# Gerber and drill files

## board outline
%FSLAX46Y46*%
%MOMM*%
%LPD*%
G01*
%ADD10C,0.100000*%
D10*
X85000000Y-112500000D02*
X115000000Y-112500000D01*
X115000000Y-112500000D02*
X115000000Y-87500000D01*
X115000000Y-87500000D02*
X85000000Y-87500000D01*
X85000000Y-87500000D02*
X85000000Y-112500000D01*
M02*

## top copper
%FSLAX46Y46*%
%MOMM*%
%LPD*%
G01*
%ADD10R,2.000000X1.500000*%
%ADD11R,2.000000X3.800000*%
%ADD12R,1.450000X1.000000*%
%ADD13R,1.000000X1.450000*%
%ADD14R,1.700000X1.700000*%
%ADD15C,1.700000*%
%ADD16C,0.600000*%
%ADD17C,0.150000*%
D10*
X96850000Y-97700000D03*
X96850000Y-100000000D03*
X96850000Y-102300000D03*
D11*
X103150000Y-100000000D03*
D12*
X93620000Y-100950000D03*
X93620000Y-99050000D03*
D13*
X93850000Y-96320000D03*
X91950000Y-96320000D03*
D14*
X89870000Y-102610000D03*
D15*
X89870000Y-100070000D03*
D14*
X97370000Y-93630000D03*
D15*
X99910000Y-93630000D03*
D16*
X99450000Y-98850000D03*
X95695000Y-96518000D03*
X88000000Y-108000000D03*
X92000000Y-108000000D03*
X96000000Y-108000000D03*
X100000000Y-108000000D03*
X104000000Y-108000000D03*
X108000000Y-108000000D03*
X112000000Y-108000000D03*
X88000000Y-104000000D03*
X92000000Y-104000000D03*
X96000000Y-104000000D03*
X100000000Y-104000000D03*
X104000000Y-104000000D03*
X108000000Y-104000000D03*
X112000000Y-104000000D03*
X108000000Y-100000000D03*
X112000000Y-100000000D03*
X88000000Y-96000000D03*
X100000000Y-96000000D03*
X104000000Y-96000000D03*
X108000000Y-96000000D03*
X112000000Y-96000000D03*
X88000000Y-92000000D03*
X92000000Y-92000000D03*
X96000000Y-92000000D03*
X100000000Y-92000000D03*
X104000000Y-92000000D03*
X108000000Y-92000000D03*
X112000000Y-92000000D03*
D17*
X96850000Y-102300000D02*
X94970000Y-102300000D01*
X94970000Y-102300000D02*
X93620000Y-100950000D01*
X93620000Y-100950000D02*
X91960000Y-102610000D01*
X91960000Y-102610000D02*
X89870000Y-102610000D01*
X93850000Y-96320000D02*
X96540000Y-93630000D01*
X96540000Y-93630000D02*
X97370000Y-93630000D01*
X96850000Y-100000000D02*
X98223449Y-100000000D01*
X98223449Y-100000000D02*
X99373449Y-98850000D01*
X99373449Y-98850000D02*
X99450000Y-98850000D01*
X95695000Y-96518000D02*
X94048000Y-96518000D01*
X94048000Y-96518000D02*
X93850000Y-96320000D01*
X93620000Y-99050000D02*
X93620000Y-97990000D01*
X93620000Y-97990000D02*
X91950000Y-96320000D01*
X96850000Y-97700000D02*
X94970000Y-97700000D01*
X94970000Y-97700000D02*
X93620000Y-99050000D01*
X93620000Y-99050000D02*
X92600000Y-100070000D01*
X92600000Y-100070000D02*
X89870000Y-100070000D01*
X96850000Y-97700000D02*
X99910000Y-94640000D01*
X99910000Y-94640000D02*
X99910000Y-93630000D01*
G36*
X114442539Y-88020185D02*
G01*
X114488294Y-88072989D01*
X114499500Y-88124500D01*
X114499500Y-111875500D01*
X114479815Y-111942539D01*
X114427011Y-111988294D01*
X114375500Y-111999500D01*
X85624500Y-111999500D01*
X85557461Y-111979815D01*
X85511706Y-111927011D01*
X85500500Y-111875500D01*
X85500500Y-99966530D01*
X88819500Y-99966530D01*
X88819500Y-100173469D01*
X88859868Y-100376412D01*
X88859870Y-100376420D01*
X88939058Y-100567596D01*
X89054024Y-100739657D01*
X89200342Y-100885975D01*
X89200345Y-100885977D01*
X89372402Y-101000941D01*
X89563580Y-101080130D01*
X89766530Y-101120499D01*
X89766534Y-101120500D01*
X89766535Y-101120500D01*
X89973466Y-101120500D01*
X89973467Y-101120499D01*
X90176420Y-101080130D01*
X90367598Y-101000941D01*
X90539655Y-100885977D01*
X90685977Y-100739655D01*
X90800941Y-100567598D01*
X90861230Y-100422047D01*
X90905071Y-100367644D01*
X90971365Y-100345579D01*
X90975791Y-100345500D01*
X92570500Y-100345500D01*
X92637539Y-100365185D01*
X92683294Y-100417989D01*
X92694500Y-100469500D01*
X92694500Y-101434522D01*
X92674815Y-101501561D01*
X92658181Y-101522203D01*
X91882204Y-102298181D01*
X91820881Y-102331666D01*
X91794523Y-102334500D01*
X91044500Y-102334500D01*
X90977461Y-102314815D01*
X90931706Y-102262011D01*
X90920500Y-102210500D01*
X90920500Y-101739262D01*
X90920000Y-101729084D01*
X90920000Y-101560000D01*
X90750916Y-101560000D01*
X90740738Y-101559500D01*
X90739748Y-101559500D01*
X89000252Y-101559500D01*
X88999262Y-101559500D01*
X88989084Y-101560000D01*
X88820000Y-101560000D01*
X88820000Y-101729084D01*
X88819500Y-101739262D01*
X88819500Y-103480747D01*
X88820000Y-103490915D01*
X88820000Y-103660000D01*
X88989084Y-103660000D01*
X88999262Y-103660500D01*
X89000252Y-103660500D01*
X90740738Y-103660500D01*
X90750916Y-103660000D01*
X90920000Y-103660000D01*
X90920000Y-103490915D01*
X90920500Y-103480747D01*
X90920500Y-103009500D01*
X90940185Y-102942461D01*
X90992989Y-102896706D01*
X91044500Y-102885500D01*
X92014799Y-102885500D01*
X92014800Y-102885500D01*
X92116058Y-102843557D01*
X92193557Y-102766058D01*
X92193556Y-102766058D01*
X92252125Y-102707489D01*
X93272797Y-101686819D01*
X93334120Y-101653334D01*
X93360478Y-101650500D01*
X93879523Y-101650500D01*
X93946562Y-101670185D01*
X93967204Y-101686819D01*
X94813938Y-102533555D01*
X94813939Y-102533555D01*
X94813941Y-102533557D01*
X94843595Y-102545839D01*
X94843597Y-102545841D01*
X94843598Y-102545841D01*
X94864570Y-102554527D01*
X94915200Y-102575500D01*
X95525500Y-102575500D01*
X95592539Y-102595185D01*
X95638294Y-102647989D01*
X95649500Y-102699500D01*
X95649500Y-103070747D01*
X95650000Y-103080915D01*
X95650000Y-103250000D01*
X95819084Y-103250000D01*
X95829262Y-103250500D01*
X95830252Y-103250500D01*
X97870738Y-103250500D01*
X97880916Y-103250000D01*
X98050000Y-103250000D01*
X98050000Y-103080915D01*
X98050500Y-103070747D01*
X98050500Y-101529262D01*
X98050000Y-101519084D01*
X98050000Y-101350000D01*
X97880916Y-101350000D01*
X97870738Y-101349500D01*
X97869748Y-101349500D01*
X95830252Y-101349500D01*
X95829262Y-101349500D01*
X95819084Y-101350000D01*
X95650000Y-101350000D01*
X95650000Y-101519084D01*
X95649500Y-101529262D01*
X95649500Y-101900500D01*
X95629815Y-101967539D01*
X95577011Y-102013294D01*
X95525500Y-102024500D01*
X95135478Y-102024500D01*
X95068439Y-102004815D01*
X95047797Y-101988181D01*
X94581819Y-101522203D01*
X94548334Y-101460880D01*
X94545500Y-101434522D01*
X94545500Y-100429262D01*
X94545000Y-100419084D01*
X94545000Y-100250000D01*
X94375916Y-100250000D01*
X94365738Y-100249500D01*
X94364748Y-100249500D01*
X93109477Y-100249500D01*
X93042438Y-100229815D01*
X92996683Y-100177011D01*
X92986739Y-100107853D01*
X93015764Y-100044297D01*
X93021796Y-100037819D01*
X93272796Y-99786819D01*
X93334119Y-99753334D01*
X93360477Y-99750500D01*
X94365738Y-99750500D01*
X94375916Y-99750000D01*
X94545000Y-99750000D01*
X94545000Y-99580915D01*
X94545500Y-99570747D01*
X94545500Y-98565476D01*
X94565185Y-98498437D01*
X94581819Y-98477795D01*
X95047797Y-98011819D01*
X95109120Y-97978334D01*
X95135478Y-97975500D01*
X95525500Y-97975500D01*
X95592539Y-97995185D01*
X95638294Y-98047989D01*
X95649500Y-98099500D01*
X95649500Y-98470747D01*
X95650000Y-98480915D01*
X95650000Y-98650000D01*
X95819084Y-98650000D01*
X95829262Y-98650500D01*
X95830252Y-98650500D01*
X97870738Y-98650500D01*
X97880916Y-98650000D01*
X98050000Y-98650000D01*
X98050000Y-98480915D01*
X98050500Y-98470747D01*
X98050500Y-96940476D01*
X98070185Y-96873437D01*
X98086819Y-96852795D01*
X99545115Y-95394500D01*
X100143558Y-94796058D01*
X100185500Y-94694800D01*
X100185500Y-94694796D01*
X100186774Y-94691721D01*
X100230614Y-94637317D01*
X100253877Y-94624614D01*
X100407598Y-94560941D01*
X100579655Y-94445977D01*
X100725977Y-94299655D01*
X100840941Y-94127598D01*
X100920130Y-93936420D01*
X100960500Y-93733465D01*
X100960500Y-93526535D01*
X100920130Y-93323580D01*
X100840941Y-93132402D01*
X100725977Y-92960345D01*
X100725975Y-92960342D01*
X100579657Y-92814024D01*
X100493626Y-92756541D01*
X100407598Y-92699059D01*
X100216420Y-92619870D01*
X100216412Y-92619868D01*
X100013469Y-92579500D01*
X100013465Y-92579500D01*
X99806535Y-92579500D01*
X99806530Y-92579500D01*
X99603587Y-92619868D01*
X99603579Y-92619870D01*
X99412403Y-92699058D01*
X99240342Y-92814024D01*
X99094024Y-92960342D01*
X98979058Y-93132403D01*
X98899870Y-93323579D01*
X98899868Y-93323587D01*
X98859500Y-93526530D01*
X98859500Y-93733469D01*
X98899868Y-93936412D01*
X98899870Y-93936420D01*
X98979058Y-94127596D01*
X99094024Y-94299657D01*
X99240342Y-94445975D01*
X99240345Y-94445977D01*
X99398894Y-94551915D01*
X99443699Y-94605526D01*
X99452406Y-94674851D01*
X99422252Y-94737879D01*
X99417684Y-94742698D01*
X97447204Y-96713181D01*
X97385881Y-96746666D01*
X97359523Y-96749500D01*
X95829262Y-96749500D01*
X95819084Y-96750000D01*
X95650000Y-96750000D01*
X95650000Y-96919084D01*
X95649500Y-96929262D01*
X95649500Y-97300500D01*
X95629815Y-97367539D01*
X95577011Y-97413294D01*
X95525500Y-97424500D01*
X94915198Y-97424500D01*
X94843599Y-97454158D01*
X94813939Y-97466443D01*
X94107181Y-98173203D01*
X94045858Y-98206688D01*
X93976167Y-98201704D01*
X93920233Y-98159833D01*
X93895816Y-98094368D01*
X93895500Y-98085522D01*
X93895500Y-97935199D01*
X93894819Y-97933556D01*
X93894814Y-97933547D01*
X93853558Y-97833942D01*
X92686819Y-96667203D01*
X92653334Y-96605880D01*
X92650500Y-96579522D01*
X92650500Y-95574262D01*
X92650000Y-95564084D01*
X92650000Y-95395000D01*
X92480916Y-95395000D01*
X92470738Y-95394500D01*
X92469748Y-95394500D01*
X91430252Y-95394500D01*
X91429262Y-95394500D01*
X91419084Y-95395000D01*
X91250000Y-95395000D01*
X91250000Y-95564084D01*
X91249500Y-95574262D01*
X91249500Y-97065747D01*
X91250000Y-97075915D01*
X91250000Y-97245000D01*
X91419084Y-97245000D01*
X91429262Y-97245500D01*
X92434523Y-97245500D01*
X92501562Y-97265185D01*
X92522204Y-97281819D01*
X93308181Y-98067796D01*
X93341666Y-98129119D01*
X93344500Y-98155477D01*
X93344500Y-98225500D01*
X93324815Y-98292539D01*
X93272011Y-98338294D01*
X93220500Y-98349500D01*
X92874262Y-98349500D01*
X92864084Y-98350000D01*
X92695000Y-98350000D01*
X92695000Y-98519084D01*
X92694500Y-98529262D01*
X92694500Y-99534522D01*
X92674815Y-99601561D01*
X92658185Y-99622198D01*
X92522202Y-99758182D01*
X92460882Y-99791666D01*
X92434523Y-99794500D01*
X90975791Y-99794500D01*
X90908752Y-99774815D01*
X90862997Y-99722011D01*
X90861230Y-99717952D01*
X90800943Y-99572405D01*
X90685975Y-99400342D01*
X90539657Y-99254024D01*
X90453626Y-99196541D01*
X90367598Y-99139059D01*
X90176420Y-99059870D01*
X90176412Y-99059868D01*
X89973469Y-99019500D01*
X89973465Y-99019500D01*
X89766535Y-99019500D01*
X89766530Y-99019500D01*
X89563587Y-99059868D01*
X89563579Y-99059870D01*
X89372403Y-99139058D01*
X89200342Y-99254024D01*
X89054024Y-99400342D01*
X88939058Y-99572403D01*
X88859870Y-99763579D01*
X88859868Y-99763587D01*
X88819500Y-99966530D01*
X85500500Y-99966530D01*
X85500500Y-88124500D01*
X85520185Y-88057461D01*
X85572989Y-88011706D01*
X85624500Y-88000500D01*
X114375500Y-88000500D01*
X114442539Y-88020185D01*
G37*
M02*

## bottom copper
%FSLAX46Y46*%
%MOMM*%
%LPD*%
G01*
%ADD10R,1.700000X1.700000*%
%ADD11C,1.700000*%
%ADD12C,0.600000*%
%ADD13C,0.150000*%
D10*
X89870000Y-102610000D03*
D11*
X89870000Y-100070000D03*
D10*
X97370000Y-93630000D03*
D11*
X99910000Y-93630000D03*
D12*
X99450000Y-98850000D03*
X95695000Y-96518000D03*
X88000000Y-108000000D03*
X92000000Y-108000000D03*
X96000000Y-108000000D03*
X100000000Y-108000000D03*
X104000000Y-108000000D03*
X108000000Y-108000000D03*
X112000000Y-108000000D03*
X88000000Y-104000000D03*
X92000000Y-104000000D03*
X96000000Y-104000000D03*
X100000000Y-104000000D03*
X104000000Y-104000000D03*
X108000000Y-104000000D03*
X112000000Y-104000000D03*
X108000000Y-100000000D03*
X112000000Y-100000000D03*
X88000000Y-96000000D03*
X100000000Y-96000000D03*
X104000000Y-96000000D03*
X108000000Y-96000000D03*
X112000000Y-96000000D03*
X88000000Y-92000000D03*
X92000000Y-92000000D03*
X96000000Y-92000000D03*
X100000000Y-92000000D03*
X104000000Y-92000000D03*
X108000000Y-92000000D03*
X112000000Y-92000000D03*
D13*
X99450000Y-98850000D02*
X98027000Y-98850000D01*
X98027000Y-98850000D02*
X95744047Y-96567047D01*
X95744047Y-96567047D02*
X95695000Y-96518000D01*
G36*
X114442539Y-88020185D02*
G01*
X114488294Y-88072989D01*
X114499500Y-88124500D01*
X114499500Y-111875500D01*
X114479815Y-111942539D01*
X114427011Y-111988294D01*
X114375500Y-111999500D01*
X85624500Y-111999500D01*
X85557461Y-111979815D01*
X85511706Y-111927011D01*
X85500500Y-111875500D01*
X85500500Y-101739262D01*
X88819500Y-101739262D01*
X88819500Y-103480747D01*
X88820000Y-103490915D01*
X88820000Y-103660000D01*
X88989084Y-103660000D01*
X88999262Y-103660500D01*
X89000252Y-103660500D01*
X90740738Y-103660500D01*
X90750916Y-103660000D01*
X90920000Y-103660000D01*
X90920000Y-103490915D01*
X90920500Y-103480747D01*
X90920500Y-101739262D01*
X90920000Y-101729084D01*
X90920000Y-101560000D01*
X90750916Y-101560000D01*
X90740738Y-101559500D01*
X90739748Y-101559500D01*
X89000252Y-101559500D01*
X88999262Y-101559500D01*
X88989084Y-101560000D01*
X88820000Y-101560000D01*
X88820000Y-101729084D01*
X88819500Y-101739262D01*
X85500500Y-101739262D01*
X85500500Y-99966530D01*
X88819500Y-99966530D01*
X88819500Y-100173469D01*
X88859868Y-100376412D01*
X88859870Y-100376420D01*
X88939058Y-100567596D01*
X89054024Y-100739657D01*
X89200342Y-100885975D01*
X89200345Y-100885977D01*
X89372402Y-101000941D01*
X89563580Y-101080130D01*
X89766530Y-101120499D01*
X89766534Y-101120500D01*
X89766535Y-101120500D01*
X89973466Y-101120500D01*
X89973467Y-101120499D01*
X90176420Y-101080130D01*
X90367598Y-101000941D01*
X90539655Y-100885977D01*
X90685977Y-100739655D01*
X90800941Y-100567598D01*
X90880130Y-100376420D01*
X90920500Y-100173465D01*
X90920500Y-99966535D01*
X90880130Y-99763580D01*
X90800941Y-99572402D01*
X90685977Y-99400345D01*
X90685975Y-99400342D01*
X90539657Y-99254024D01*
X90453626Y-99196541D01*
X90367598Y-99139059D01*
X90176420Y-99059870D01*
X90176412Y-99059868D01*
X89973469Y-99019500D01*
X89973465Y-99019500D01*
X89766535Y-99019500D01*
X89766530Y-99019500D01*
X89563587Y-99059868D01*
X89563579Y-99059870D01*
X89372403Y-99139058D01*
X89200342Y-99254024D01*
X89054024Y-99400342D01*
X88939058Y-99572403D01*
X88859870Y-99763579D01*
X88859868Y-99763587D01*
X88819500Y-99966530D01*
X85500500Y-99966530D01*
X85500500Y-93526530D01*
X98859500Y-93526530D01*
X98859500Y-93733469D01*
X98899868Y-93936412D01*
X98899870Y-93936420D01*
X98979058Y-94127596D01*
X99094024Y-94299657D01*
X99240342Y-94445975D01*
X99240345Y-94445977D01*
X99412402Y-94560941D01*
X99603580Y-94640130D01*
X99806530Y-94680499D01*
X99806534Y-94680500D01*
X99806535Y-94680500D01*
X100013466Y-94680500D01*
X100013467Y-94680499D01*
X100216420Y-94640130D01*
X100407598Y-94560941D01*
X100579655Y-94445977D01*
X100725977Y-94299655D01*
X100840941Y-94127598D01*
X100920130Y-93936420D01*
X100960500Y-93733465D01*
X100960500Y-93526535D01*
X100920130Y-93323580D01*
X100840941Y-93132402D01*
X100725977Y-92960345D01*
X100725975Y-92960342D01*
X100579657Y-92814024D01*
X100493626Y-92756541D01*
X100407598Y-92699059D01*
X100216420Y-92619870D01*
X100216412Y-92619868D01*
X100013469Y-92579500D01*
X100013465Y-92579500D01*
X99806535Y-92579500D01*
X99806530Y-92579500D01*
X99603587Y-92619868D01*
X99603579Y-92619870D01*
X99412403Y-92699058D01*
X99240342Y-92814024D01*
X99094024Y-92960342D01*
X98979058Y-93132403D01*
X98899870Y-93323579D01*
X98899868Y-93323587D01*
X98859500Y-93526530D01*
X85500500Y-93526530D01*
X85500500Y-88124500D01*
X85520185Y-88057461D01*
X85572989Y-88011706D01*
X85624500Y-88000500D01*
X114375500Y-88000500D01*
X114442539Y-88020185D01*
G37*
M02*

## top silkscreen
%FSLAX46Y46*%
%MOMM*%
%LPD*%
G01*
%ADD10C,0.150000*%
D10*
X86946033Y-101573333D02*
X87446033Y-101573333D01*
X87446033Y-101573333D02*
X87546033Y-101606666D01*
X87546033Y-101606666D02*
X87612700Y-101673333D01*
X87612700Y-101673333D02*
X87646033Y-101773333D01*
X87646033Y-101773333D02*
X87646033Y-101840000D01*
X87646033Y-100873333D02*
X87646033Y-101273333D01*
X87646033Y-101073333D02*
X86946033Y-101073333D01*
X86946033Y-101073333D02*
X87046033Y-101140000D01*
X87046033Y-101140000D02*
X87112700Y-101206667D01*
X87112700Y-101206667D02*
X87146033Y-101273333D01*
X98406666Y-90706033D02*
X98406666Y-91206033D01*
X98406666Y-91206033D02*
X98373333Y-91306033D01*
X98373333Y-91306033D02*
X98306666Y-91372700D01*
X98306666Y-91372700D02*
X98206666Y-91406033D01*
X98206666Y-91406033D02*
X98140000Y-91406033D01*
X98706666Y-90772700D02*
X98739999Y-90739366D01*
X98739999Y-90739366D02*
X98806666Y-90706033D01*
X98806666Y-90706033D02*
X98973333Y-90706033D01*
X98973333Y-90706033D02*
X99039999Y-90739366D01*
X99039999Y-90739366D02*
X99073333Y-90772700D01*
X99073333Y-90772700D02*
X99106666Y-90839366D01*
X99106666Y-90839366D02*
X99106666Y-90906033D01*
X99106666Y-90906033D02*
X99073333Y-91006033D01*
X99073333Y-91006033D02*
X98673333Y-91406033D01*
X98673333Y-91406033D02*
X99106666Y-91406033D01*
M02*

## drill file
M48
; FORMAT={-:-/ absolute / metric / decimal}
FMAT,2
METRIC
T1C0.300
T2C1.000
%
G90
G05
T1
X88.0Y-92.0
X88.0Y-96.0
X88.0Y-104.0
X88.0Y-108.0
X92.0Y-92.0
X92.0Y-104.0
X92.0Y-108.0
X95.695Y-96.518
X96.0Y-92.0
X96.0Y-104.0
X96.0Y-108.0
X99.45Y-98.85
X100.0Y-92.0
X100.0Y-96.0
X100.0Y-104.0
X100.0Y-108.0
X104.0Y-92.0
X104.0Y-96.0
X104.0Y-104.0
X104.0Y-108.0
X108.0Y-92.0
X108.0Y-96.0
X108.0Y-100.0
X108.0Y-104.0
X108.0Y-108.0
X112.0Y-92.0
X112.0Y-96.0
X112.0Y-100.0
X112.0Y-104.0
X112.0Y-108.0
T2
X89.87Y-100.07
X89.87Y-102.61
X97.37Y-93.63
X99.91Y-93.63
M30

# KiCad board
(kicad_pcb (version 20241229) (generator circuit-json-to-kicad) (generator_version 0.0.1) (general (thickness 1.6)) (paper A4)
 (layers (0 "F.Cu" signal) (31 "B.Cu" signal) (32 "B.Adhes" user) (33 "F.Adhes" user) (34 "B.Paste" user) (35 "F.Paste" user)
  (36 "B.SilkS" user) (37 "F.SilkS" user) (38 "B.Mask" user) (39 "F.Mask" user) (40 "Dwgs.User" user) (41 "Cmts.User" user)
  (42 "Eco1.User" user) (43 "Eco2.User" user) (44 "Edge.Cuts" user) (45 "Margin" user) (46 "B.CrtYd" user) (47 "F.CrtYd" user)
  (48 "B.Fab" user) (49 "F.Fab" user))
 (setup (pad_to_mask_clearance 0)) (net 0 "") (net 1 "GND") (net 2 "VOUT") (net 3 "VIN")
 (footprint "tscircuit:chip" (layer F.Cu) (at 100 100 0)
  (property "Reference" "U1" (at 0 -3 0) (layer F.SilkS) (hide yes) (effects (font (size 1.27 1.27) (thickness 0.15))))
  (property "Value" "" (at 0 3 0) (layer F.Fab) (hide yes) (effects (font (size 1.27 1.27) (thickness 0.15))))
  (pad "1" smd rect (at -3.15 -2.3 0) (size 2 1.5) (layers F.Cu F.Mask) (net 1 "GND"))
  (pad "2" smd rect (at -3.15 0 0) (size 2 1.5) (layers F.Cu F.Mask) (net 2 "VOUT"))
  (pad "3" smd rect (at -3.15 2.3 0) (size 2 1.5) (layers F.Cu F.Mask) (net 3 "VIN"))
  (pad "2" smd rect (at 3.15 0 0) (size 2 3.8) (layers F.Cu F.Mask) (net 2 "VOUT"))
  (pad "" smd rect (at -3.15 -2.3 0) (size 1.4 1.0499999999999998) (layers F.Paste))
  (pad "" smd rect (at -3.15 0 0) (size 1.4 1.0499999999999998) (layers F.Paste))
  (pad "" smd rect (at -3.15 2.3 0) (size 1.4 1.0499999999999998) (layers F.Paste))
  (pad "" smd rect (at 3.15 0 0) (size 1.4 2.6599999999999997) (layers F.Paste)))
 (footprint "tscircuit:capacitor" (layer F.Cu) (at 93.62 100 90)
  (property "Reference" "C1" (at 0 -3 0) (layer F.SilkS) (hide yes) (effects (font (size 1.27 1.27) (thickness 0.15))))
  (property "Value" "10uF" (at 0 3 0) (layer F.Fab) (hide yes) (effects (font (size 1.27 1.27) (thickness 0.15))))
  (pad "1" smd rect (at -0.95 0 0) (size 1.45 1) (layers F.Cu F.Mask) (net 3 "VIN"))
  (pad "2" smd rect (at 0.95 0 0) (size 1.45 1) (layers F.Cu F.Mask) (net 1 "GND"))
  (pad "" smd rect (at -0.95 0 0) (size 1.015 0.7) (layers F.Paste))
  (pad "" smd rect (at 0.95 0 0) (size 1.015 0.7) (layers F.Paste)))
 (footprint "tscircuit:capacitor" (layer F.Cu) (at 92.9 96.32 180)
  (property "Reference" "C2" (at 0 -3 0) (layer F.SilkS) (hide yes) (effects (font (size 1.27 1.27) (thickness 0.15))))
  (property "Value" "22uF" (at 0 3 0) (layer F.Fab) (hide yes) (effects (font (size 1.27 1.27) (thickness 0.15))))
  (pad "1" smd rect (at -0.9500000000000002 0 0) (size 1 1.45) (layers F.Cu F.Mask) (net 2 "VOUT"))
  (pad "2" smd rect (at 0.9499999999999993 0 0) (size 1 1.45) (layers F.Cu F.Mask) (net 1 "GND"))
  (pad "" smd rect (at -0.9500000000000002 0 0) (size 0.7 1.015) (layers F.Paste))
  (pad "" smd rect (at 0.9499999999999993 0 0) (size 0.7 1.015) (layers F.Paste)))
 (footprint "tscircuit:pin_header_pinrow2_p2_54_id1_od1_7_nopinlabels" (layer F.Cu) (at 89.87 101.34 90)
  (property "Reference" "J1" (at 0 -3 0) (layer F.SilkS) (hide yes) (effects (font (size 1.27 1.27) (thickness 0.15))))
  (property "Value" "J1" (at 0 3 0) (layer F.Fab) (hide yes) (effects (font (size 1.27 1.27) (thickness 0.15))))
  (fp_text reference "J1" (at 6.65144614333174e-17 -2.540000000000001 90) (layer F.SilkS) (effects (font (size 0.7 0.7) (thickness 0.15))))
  (pad "1" thru_hole rect (at -1.27 7.776507174585693e-17 90) (size 1.7 1.7) (drill 1) (layers *.Cu *.Mask) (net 3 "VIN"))
  (pad "2" thru_hole circle (at 1.27 -7.776507174585693e-17 0) (size 1.7 1.7) (drill 1) (layers *.Cu *.Mask) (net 1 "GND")))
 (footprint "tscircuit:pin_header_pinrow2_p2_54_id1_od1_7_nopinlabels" (layer F.Cu) (at 98.64 93.63 0)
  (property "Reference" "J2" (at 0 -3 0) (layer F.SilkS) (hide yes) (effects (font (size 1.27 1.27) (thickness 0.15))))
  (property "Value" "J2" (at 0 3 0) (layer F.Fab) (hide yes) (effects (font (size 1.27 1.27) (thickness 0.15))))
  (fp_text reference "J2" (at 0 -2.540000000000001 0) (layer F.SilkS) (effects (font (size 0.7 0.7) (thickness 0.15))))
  (pad "1" thru_hole rect (at -1.27 0 0) (size 1.7 1.7) (drill 1) (layers *.Cu *.Mask) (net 2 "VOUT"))
  (pad "2" thru_hole circle (at 1.27 0 0) (size 1.7 1.7) (drill 1) (layers *.Cu *.Mask) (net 1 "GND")))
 (segment (start 96.85 102.3) (end 94.97 102.3) (width 0.15) (layer F.Cu) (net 3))
 (segment (start 94.97 102.3) (end 93.62 100.95) (width 0.15) (layer F.Cu) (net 3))
 (segment (start 93.62 100.95) (end 91.96 102.61) (width 0.15) (layer F.Cu) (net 3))
 (segment (start 91.96 102.61) (end 89.87 102.61) (width 0.15) (layer F.Cu) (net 3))
 (segment (start 93.85 96.32) (end 96.53999999999999 93.63) (width 0.15) (layer F.Cu) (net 2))
 (segment (start 96.53999999999999 93.63) (end 97.37 93.63) (width 0.15) (layer F.Cu) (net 2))
 (segment (start 96.85 100) (end 98.22344899188154 100) (width 0.15) (layer F.Cu) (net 2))
 (segment (start 98.22344899188154 100) (end 99.37344899188153 98.85) (width 0.15) (layer F.Cu) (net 2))
 (segment (start 99.37344899188153 98.85) (end 99.45 98.85) (width 0.15) (layer F.Cu) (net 2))
 (segment (start 99.45 98.85) (end 98.027 98.85) (width 0.15) (layer B.Cu) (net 2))
 (segment (start 98.027 98.85) (end 95.74404689936635 96.56704689936635) (width 0.15) (layer B.Cu) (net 2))
 (segment (start 95.74404689936635 96.56704689936635) (end 95.695 96.518) (width 0.15) (layer B.Cu) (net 2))
 (segment (start 95.695 96.518) (end 94.048 96.518) (width 0.15) (layer F.Cu) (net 2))
 (segment (start 94.048 96.518) (end 93.85 96.32) (width 0.15) (layer F.Cu) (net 2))
 (segment (start 93.62 99.05) (end 93.62 97.99) (width 0.15) (layer F.Cu) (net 1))
 (segment (start 93.62 97.99) (end 91.95 96.32) (width 0.15) (layer F.Cu) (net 1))
 (segment (start 96.85 97.7) (end 94.97 97.7) (width 0.15) (layer F.Cu) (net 1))
 (segment (start 94.97 97.7) (end 93.62 99.05) (width 0.15) (layer F.Cu) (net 1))
 (segment (start 93.62 99.05) (end 92.6 100.07000000000001) (width 0.15) (layer F.Cu) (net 1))
 (segment (start 92.6 100.07000000000001) (end 89.87 100.07000000000001) (width 0.15) (layer F.Cu) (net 1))
 (segment (start 96.85 97.7) (end 99.91 94.64) (width 0.15) (layer F.Cu) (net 1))
 (segment (start 99.91 94.64) (end 99.91 93.63) (width 0.15) (layer F.Cu) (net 1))
 (gr_line (start 85 112.5) (end 115 112.5) (width 0.1) (layer Edge.Cuts))
 (gr_line (start 115 112.5) (end 115 87.5) (width 0.1) (layer Edge.Cuts))
 (gr_line (start 115 87.5) (end 85 87.5) (width 0.1) (layer Edge.Cuts))
 (gr_line (start 85 87.5) (end 85 112.5) (width 0.1) (layer Edge.Cuts))
 (via (at 99.45 98.85) (size 0.6) (drill 0.3) (layers F.Cu B.Cu) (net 2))
 (via (at 95.695 96.518) (size 0.6) (drill 0.3) (layers F.Cu B.Cu) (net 2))
 (via (at 88 108) (size 0.6) (drill 0.3) (layers F.Cu B.Cu) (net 2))
 (via (at 92 108) (size 0.6) (drill 0.3) (layers F.Cu B.Cu) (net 2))
 (via (at 96 108) (size 0.6) (drill 0.3) (layers F.Cu B.Cu) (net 2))
 (via (at 100 108) (size 0.6) (drill 0.3) (layers F.Cu B.Cu) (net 2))
 (via (at 104 108) (size 0.6) (drill 0.3) (layers F.Cu B.Cu) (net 2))
 (via (at 108 108) (size 0.6) (drill 0.3) (layers F.Cu B.Cu) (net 2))
 (via (at 112 108) (size 0.6) (drill 0.3) (layers F.Cu B.Cu) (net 2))
 (via (at 88 104) (size 0.6) (drill 0.3) (layers F.Cu B.Cu) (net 2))
 (via (at 92 104) (size 0.6) (drill 0.3) (layers F.Cu B.Cu) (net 2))
 (via (at 96 104) (size 0.6) (drill 0.3) (layers F.Cu B.Cu) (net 2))
 (via (at 100 104) (size 0.6) (drill 0.3) (layers F.Cu B.Cu) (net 2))
 (via (at 104 104) (size 0.6) (drill 0.3) (layers F.Cu B.Cu) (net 2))
 (via (at 108 104) (size 0.6) (drill 0.3) (layers F.Cu B.Cu) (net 2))
 (via (at 112 104) (size 0.6) (drill 0.3) (layers F.Cu B.Cu) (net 2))
 (via (at 108 100) (size 0.6) (drill 0.3) (layers F.Cu B.Cu) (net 2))
 (via (at 112 100) (size 0.6) (drill 0.3) (layers F.Cu B.Cu) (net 2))
 (via (at 88 96) (size 0.6) (drill 0.3) (layers F.Cu B.Cu) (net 2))
 (via (at 100 96) (size 0.6) (drill 0.3) (layers F.Cu B.Cu) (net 2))
 (via (at 104 96) (size 0.6) (drill 0.3) (layers F.Cu B.Cu) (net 2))
 (via (at 108 96) (size 0.6) (drill 0.3) (layers F.Cu B.Cu) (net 2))
 (via (at 112 96) (size 0.6) (drill 0.3) (layers F.Cu B.Cu) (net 2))
 (via (at 88 92) (size 0.6) (drill 0.3) (layers F.Cu B.Cu) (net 2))
 (via (at 92 92) (size 0.6) (drill 0.3) (layers F.Cu B.Cu) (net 2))
 (via (at 96 92) (size 0.6) (drill 0.3) (layers F.Cu B.Cu) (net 2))
 (via (at 100 92) (size 0.6) (drill 0.3) (layers F.Cu B.Cu) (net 2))
 (via (at 104 92) (size 0.6) (drill 0.3) (layers F.Cu B.Cu) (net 2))
 (via (at 108 92) (size 0.6) (drill 0.3) (layers F.Cu B.Cu) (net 2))
 (via (at 112 92) (size 0.6) (drill 0.3) (layers F.Cu B.Cu) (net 2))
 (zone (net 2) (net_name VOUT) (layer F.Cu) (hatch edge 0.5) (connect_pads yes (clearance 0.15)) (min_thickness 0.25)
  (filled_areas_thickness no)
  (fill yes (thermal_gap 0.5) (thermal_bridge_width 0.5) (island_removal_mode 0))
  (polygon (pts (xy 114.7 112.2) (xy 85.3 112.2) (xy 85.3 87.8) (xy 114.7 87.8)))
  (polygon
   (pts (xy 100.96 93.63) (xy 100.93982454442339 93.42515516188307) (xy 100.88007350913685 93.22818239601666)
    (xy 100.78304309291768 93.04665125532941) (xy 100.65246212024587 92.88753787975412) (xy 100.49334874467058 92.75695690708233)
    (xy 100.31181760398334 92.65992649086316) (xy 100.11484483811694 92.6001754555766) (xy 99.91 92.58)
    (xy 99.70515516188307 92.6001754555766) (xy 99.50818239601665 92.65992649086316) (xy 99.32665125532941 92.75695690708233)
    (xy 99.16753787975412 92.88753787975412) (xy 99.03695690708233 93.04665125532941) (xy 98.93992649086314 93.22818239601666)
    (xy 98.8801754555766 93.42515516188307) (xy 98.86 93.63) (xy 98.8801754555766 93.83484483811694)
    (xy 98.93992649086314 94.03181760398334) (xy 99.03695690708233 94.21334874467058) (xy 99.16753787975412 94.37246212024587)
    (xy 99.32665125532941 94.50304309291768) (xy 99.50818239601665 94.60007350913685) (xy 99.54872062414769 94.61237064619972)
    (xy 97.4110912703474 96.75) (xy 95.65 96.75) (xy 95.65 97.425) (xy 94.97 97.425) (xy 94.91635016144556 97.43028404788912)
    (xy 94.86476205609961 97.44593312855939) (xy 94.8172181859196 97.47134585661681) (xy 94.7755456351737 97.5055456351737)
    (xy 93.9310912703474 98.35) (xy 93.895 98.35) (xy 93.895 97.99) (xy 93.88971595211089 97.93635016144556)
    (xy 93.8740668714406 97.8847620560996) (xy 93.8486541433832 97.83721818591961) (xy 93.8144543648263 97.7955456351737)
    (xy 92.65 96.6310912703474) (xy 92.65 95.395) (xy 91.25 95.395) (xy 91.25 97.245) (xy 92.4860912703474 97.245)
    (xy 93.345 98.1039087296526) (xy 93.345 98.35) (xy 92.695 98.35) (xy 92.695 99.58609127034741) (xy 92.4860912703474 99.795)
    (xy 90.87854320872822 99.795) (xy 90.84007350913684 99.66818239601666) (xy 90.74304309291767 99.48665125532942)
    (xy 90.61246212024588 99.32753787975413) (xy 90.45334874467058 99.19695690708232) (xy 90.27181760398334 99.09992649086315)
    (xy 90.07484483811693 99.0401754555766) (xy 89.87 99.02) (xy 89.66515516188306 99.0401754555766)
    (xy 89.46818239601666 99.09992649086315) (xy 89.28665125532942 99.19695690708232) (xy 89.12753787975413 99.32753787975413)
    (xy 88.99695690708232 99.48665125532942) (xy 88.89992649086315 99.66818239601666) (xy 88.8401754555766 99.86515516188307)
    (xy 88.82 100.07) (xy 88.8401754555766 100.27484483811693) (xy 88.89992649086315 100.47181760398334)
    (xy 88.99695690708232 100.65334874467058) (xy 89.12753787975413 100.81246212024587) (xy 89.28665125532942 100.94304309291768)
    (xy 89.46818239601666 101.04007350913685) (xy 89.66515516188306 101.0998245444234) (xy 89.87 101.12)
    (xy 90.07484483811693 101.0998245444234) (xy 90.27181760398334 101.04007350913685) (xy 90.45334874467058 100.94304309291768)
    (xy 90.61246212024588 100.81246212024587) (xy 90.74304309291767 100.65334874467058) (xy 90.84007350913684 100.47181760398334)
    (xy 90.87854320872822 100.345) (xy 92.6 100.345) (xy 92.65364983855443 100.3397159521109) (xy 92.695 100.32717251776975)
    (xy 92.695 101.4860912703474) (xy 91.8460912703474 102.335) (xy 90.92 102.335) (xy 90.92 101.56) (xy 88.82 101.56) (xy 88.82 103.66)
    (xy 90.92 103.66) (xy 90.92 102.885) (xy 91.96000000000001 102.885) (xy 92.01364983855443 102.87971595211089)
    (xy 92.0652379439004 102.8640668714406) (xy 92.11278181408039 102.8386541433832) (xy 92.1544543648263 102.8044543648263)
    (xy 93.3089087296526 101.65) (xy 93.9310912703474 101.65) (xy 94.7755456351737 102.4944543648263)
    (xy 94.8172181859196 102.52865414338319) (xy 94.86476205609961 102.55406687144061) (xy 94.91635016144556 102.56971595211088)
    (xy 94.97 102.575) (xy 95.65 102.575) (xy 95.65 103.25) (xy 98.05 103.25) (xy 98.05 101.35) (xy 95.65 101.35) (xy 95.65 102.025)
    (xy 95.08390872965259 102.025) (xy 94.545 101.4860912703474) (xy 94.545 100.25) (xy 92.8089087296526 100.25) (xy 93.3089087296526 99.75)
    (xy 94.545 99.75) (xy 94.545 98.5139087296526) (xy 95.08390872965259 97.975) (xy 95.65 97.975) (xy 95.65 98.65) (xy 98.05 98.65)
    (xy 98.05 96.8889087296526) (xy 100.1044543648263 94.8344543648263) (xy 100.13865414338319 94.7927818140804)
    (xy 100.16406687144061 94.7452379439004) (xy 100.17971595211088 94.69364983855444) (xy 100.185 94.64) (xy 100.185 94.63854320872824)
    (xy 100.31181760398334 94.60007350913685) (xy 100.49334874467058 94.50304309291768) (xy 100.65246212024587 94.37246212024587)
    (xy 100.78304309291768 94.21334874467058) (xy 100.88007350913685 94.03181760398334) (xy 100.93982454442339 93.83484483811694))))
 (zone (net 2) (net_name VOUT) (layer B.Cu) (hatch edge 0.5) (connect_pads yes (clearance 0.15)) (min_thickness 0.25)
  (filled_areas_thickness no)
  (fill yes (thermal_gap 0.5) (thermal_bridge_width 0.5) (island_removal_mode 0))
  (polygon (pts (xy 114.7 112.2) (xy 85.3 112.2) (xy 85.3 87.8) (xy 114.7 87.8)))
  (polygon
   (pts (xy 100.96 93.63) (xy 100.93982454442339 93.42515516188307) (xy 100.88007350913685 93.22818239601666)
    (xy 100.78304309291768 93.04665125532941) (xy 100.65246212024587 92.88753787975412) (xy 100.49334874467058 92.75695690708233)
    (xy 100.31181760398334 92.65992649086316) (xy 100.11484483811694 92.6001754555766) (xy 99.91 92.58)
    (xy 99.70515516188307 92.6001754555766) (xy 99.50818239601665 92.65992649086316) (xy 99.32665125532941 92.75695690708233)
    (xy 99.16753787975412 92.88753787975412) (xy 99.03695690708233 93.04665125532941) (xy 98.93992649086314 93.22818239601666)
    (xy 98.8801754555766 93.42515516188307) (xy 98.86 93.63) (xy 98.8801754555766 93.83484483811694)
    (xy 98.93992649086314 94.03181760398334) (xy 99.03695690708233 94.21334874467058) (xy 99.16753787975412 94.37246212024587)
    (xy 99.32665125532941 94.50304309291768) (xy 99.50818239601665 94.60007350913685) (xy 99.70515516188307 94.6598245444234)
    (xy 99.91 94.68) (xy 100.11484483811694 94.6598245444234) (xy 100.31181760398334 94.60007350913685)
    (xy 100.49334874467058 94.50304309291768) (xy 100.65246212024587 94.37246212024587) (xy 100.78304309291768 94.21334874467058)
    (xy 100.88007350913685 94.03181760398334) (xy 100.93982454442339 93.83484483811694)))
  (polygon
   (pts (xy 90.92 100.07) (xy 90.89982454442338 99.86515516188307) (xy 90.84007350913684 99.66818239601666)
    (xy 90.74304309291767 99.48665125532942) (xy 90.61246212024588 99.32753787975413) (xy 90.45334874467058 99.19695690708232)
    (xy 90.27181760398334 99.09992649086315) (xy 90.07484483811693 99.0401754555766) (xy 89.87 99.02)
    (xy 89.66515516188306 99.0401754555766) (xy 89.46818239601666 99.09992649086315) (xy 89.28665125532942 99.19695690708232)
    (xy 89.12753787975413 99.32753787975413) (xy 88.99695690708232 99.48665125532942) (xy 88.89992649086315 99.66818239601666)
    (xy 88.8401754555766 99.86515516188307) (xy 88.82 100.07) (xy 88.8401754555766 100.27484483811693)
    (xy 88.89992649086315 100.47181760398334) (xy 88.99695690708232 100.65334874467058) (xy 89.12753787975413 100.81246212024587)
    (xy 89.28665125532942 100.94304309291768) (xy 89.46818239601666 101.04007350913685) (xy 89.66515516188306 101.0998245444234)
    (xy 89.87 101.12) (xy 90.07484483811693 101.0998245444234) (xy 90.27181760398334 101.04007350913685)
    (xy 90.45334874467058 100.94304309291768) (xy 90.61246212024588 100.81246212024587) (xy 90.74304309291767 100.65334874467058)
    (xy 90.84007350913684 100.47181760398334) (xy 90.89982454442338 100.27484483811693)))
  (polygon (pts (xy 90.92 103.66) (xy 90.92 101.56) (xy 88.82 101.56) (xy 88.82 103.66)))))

